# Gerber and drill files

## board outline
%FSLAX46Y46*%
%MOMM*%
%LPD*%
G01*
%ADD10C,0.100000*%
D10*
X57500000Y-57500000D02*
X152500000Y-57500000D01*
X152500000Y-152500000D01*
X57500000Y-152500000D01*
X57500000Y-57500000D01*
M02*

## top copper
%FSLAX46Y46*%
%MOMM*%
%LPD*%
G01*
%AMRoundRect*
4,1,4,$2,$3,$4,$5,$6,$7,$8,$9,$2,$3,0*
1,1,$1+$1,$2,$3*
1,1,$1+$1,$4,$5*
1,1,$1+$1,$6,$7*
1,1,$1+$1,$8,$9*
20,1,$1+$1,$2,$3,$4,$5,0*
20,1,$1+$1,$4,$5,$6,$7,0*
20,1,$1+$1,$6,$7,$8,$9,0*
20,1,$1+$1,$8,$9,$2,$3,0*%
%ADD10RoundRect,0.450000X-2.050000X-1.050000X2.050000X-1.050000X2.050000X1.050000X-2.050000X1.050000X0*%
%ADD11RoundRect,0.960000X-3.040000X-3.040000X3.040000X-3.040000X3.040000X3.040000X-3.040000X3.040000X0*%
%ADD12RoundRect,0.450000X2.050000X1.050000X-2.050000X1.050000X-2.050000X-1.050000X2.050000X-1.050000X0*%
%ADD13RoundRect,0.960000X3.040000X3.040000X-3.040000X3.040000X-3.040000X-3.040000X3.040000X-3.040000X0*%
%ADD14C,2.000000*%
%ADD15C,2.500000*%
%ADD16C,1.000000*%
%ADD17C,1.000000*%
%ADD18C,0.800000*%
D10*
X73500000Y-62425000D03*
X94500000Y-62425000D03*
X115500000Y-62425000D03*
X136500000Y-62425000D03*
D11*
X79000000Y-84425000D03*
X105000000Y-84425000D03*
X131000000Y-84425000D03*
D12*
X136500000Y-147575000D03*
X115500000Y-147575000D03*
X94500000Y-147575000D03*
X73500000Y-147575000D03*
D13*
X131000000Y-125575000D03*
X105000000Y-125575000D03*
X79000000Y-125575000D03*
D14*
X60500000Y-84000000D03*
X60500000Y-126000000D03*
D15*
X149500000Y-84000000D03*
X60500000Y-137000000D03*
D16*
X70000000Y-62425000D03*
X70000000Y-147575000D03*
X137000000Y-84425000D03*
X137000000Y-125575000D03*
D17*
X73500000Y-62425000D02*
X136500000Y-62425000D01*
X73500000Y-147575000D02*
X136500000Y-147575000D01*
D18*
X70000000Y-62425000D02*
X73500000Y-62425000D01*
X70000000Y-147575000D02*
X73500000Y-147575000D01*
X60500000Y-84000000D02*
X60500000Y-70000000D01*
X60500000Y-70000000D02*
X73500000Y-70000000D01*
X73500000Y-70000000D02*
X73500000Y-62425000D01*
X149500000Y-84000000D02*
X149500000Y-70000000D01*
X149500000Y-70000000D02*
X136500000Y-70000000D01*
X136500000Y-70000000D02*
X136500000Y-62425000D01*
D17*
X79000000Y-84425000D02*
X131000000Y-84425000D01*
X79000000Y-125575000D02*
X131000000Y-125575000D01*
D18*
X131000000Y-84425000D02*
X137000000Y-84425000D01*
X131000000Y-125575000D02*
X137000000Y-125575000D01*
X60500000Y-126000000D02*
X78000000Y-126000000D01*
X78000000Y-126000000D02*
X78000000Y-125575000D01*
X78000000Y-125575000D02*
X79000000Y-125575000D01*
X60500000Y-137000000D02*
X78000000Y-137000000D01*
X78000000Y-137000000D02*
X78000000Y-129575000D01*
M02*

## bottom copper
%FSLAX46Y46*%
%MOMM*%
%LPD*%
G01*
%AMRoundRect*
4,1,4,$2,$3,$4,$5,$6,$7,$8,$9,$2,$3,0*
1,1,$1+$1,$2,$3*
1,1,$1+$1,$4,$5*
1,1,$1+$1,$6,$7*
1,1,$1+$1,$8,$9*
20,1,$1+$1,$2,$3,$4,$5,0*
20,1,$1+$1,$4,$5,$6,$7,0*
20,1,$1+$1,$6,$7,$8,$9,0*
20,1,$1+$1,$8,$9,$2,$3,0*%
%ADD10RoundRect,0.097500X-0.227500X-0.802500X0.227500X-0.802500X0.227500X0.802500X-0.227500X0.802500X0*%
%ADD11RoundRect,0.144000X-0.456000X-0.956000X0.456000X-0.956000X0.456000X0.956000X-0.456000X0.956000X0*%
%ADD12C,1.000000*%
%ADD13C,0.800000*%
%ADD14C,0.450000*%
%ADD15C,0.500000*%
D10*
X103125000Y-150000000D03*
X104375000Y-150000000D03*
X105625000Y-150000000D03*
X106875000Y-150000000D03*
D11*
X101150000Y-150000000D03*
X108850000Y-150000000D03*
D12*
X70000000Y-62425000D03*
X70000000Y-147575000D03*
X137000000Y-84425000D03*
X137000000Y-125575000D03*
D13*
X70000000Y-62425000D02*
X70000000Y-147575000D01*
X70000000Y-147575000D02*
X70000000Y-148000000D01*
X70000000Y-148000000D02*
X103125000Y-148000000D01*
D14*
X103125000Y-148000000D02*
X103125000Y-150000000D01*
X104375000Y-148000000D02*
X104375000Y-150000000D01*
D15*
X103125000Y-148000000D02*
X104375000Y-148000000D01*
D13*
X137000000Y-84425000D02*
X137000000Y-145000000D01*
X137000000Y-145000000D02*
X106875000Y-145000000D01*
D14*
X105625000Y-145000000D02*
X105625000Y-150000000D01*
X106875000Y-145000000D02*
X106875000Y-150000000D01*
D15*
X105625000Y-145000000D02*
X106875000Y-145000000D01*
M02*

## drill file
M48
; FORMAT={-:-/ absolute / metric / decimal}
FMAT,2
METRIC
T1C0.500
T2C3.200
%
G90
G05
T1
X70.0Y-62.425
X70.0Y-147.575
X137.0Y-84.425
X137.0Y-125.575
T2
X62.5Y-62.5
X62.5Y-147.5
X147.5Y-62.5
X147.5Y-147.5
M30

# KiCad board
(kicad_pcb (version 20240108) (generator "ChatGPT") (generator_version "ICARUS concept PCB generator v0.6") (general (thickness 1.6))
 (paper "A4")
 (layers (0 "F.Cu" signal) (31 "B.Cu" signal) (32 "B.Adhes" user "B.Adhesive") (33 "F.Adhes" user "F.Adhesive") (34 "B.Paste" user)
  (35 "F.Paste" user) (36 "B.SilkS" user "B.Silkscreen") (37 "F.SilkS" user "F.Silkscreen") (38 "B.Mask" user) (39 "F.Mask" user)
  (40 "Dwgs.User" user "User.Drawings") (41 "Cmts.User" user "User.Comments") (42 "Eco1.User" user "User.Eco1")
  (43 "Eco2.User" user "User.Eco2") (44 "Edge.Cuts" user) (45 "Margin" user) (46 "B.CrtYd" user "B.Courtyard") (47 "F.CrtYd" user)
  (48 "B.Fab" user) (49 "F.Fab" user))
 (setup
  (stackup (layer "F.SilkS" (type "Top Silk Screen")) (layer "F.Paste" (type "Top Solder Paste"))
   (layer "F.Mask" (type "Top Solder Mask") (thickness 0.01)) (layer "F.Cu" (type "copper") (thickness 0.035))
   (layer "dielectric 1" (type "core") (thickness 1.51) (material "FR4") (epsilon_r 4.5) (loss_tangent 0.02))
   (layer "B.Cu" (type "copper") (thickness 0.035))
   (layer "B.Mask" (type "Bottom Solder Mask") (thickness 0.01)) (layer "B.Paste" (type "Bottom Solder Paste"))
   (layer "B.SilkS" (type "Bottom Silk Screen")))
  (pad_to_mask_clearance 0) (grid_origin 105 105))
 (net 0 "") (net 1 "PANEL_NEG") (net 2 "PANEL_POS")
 (gr_rect (start 57.5 57.5) (end 152.5 152.5) (stroke (width 0.1) (type solid)) (fill none) (layer "Edge.Cuts"))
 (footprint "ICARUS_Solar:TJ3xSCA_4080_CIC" (layer "F.Cu") (at 105 84.425 0)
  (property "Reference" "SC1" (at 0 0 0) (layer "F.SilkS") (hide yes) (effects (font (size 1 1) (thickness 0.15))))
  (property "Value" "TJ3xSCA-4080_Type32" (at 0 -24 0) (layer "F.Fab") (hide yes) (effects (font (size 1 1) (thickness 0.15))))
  (pad "1" smd roundrect (at -31.5 -22.0) (size 5.0 3.0) (layers "F.Cu" "F.Mask" "F.Paste") (roundrect_rratio 0.15) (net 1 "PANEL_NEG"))
  (pad "1" smd roundrect (at -10.5 -22.0) (size 5.0 3.0) (layers "F.Cu" "F.Mask" "F.Paste") (roundrect_rratio 0.15) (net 1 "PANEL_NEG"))
  (pad "1" smd roundrect (at 10.5 -22.0) (size 5.0 3.0) (layers "F.Cu" "F.Mask" "F.Paste") (roundrect_rratio 0.15) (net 1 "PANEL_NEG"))
  (pad "1" smd roundrect (at 31.5 -22.0) (size 5.0 3.0) (layers "F.Cu" "F.Mask" "F.Paste") (roundrect_rratio 0.15) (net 1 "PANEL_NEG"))
  (pad "2" smd roundrect (at -26.0 0) (size 8.0 8.0) (layers "F.Cu" "F.Mask") (roundrect_rratio 0.12) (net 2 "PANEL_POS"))
  (pad "2" smd roundrect (at 0 0) (size 8.0 8.0) (layers "F.Cu" "F.Mask") (roundrect_rratio 0.12) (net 2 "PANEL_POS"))
  (pad "2" smd roundrect (at 26.0 0) (size 8.0 8.0) (layers "F.Cu" "F.Mask") (roundrect_rratio 0.12) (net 2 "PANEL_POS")))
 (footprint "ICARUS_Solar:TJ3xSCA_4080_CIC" (layer "F.Cu") (at 105 125.575 180)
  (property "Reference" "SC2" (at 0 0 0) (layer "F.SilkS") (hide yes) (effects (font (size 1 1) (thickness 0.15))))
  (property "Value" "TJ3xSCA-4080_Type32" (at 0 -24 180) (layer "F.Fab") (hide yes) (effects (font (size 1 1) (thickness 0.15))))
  (pad "1" smd roundrect (at -31.5 -22.0 180) (size 5.0 3.0) (layers "F.Cu" "F.Mask" "F.Paste") (roundrect_rratio 0.15) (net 1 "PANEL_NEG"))
  (pad "1" smd roundrect (at -10.5 -22.0 180) (size 5.0 3.0) (layers "F.Cu" "F.Mask" "F.Paste") (roundrect_rratio 0.15) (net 1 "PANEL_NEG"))
  (pad "1" smd roundrect (at 10.5 -22.0 180) (size 5.0 3.0) (layers "F.Cu" "F.Mask" "F.Paste") (roundrect_rratio 0.15) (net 1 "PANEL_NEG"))
  (pad "1" smd roundrect (at 31.5 -22.0 180) (size 5.0 3.0) (layers "F.Cu" "F.Mask" "F.Paste") (roundrect_rratio 0.15) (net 1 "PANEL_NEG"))
  (pad "2" smd roundrect (at -26.0 0 180) (size 8.0 8.0) (layers "F.Cu" "F.Mask") (roundrect_rratio 0.12) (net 2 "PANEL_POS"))
  (pad "2" smd roundrect (at 0 0 180) (size 8.0 8.0) (layers "F.Cu" "F.Mask") (roundrect_rratio 0.12) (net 2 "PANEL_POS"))
  (pad "2" smd roundrect (at 26.0 0 180) (size 8.0 8.0) (layers "F.Cu" "F.Mask") (roundrect_rratio 0.12) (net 2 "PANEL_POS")))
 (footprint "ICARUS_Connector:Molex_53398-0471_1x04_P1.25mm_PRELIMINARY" (layer "B.Cu") (at 105 150 0)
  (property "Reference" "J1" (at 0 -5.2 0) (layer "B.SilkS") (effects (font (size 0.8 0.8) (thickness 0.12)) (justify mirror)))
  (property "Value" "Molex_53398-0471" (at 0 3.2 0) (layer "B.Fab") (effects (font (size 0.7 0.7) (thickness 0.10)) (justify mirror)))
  (pad "1" smd roundrect (at -1.875 0) (size 0.65 1.8) (layers "B.Cu" "B.Mask" "B.Paste") (roundrect_rratio 0.15) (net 1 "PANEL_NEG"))
  (pad "2" smd roundrect (at -0.625 0) (size 0.65 1.8) (layers "B.Cu" "B.Mask" "B.Paste") (roundrect_rratio 0.15) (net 1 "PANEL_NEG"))
  (pad "3" smd roundrect (at 0.625 0) (size 0.65 1.8) (layers "B.Cu" "B.Mask" "B.Paste") (roundrect_rratio 0.15) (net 2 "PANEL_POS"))
  (pad "4" smd roundrect (at 1.875 0) (size 0.65 1.8) (layers "B.Cu" "B.Mask" "B.Paste") (roundrect_rratio 0.15) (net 2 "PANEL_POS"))
  (pad "MP1" smd roundrect (at -3.85 0) (size 1.2 2.2) (layers "B.Cu" "B.Mask" "B.Paste") (roundrect_rratio 0.12))
  (pad "MP2" smd roundrect (at 3.85 0) (size 1.2 2.2) (layers "B.Cu" "B.Mask" "B.Paste") (roundrect_rratio 0.12)))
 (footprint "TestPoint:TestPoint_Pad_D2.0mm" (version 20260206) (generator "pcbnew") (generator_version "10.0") (layer "F.Cu")
  (at 60.5 84 0)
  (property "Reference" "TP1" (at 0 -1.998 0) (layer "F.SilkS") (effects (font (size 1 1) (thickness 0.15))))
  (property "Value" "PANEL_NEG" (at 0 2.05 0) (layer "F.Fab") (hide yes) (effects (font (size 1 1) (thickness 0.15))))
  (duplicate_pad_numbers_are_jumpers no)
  (pad "1" smd circle (at 0 0) (size 2 2) (layers "F.Cu" "F.Mask") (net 1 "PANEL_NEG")))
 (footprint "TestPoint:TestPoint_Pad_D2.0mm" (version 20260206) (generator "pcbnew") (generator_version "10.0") (layer "F.Cu")
  (at 60.5 126 0)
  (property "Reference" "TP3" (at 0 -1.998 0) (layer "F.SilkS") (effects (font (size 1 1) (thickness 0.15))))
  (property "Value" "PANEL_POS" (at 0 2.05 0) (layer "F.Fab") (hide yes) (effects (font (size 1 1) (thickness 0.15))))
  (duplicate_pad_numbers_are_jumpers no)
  (pad "1" smd circle (at 0 0) (size 2 2) (layers "F.Cu" "F.Mask") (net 2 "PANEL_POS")))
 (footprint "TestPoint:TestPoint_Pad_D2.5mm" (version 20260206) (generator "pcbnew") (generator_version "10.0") (layer "F.Cu")
  (at 149.5 84 0)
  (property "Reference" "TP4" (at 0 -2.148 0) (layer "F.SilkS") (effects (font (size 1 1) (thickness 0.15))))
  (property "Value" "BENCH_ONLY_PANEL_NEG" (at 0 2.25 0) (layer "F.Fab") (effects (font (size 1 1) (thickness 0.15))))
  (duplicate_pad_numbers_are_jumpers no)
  (pad "1" smd circle (at 0 0) (size 2.5 2.5) (layers "F.Cu" "F.Mask") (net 1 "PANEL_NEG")))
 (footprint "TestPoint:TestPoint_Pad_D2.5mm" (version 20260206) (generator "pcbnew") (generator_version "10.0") (layer "F.Cu")
  (at 60.5 137 0)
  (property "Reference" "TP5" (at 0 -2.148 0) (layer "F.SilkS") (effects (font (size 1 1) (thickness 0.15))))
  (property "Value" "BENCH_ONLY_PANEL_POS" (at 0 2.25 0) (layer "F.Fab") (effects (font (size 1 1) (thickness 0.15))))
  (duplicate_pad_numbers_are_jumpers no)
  (pad "1" smd circle (at 0 0) (size 2.5 2.5) (layers "F.Cu" "F.Mask") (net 2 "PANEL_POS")))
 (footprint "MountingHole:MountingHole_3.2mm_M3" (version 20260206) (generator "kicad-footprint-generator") (layer "F.Cu") (at 62.5 62.5)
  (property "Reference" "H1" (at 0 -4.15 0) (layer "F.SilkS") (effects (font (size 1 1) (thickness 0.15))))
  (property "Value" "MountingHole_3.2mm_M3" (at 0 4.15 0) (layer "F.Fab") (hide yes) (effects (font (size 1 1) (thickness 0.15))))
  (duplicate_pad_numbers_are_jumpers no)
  (pad "" np_thru_hole circle (at 0 0) (size 3.2 3.2) (drill 3.2) (layers "*.Cu" "*.Mask")))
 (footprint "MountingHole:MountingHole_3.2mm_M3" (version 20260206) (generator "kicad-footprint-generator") (layer "F.Cu") (at 147.5 62.5)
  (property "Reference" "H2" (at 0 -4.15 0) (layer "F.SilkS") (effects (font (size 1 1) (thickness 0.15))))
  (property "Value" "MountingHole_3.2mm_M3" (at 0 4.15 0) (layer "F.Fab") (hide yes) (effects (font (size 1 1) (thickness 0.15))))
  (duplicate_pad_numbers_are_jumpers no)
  (pad "" np_thru_hole circle (at 0 0) (size 3.2 3.2) (drill 3.2) (layers "*.Cu" "*.Mask")))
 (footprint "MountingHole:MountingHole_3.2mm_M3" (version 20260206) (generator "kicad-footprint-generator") (layer "F.Cu") (at 62.5 147.5)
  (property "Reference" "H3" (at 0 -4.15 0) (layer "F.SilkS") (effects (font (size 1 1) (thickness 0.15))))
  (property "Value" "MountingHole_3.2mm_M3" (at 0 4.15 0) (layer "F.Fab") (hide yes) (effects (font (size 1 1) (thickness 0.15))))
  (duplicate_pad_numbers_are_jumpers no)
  (pad "" np_thru_hole circle (at 0 0) (size 3.2 3.2) (drill 3.2) (layers "*.Cu" "*.Mask")))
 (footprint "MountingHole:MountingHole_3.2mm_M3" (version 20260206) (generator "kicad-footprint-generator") (layer "F.Cu") (at 147.5 147.5)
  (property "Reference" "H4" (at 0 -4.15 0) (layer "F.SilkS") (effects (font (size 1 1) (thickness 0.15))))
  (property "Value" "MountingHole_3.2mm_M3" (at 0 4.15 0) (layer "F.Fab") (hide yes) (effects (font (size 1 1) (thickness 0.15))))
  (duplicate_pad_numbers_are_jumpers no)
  (pad "" np_thru_hole circle (at 0 0) (size 3.2 3.2) (drill 3.2) (layers "*.Cu" "*.Mask")))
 (segment (start 73.5 62.425) (end 136.5 62.425) (width 1.0) (layer "F.Cu") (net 1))
 (segment (start 73.5 147.575) (end 136.5 147.575) (width 1.0) (layer "F.Cu") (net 1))
 (segment (start 70 62.425) (end 73.5 62.425) (width 0.8) (layer "F.Cu") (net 1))
 (segment (start 70 147.575) (end 73.5 147.575) (width 0.8) (layer "F.Cu") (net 1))
 (via (at 70 62.425) (size 1.0) (drill 0.5) (layers "F.Cu" "B.Cu") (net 1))
 (via (at 70 147.575) (size 1.0) (drill 0.5) (layers "F.Cu" "B.Cu") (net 1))
 (segment (start 70 62.425) (end 70 147.575) (width 0.8) (layer "B.Cu") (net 1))
 (segment (start 70 147.575) (end 70 148.0) (width 0.8) (layer "B.Cu") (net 1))
 (segment (start 70 148.0) (end 103.125 148.0) (width 0.8) (layer "B.Cu") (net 1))
 (segment (start 103.125 148.0) (end 103.125 150) (width 0.45) (layer "B.Cu") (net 1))
 (segment (start 104.375 148.0) (end 104.375 150) (width 0.45) (layer "B.Cu") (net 1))
 (segment (start 103.125 148.0) (end 104.375 148.0) (width 0.5) (layer "B.Cu") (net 1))
 (segment (start 60.5 84) (end 60.5 70) (width 0.8) (layer "F.Cu") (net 1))
 (segment (start 60.5 70) (end 73.5 70) (width 0.8) (layer "F.Cu") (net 1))
 (segment (start 73.5 70) (end 73.5 62.425) (width 0.8) (layer "F.Cu") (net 1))
 (segment (start 149.5 84) (end 149.5 70) (width 0.8) (layer "F.Cu") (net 1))
 (segment (start 149.5 70) (end 136.5 70) (width 0.8) (layer "F.Cu") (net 1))
 (segment (start 136.5 70) (end 136.5 62.425) (width 0.8) (layer "F.Cu") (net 1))
 (segment (start 79 84.425) (end 131 84.425) (width 1.0) (layer "F.Cu") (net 2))
 (segment (start 79 125.575) (end 131 125.575) (width 1.0) (layer "F.Cu") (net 2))
 (segment (start 131 84.425) (end 137 84.425) (width 0.8) (layer "F.Cu") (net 2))
 (segment (start 131 125.575) (end 137 125.575) (width 0.8) (layer "F.Cu") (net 2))
 (via (at 137 84.425) (size 1.0) (drill 0.5) (layers "F.Cu" "B.Cu") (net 2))
 (via (at 137 125.575) (size 1.0) (drill 0.5) (layers "F.Cu" "B.Cu") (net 2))
 (segment (start 137 84.425) (end 137 145) (width 0.8) (layer "B.Cu") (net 2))
 (segment (start 137 145) (end 106.875 145) (width 0.8) (layer "B.Cu") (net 2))
 (segment (start 105.625 145) (end 105.625 150) (width 0.45) (layer "B.Cu") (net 2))
 (segment (start 106.875 145) (end 106.875 150) (width 0.45) (layer "B.Cu") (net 2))
 (segment (start 105.625 145) (end 106.875 145) (width 0.5) (layer "B.Cu") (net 2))
 (segment (start 60.5 126) (end 78 126) (width 0.8) (layer "F.Cu") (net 2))
 (segment (start 78 126) (end 78 125.575) (width 0.8) (layer "F.Cu") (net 2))
 (segment (start 78 125.575) (end 79 125.575) (width 0.8) (layer "F.Cu") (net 2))
 (segment (start 60.5 137) (end 78 137) (width 0.8) (layer "F.Cu") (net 2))
 (segment (start 78 137) (end 78 129.575) (width 0.8) (layer "F.Cu") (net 2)))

